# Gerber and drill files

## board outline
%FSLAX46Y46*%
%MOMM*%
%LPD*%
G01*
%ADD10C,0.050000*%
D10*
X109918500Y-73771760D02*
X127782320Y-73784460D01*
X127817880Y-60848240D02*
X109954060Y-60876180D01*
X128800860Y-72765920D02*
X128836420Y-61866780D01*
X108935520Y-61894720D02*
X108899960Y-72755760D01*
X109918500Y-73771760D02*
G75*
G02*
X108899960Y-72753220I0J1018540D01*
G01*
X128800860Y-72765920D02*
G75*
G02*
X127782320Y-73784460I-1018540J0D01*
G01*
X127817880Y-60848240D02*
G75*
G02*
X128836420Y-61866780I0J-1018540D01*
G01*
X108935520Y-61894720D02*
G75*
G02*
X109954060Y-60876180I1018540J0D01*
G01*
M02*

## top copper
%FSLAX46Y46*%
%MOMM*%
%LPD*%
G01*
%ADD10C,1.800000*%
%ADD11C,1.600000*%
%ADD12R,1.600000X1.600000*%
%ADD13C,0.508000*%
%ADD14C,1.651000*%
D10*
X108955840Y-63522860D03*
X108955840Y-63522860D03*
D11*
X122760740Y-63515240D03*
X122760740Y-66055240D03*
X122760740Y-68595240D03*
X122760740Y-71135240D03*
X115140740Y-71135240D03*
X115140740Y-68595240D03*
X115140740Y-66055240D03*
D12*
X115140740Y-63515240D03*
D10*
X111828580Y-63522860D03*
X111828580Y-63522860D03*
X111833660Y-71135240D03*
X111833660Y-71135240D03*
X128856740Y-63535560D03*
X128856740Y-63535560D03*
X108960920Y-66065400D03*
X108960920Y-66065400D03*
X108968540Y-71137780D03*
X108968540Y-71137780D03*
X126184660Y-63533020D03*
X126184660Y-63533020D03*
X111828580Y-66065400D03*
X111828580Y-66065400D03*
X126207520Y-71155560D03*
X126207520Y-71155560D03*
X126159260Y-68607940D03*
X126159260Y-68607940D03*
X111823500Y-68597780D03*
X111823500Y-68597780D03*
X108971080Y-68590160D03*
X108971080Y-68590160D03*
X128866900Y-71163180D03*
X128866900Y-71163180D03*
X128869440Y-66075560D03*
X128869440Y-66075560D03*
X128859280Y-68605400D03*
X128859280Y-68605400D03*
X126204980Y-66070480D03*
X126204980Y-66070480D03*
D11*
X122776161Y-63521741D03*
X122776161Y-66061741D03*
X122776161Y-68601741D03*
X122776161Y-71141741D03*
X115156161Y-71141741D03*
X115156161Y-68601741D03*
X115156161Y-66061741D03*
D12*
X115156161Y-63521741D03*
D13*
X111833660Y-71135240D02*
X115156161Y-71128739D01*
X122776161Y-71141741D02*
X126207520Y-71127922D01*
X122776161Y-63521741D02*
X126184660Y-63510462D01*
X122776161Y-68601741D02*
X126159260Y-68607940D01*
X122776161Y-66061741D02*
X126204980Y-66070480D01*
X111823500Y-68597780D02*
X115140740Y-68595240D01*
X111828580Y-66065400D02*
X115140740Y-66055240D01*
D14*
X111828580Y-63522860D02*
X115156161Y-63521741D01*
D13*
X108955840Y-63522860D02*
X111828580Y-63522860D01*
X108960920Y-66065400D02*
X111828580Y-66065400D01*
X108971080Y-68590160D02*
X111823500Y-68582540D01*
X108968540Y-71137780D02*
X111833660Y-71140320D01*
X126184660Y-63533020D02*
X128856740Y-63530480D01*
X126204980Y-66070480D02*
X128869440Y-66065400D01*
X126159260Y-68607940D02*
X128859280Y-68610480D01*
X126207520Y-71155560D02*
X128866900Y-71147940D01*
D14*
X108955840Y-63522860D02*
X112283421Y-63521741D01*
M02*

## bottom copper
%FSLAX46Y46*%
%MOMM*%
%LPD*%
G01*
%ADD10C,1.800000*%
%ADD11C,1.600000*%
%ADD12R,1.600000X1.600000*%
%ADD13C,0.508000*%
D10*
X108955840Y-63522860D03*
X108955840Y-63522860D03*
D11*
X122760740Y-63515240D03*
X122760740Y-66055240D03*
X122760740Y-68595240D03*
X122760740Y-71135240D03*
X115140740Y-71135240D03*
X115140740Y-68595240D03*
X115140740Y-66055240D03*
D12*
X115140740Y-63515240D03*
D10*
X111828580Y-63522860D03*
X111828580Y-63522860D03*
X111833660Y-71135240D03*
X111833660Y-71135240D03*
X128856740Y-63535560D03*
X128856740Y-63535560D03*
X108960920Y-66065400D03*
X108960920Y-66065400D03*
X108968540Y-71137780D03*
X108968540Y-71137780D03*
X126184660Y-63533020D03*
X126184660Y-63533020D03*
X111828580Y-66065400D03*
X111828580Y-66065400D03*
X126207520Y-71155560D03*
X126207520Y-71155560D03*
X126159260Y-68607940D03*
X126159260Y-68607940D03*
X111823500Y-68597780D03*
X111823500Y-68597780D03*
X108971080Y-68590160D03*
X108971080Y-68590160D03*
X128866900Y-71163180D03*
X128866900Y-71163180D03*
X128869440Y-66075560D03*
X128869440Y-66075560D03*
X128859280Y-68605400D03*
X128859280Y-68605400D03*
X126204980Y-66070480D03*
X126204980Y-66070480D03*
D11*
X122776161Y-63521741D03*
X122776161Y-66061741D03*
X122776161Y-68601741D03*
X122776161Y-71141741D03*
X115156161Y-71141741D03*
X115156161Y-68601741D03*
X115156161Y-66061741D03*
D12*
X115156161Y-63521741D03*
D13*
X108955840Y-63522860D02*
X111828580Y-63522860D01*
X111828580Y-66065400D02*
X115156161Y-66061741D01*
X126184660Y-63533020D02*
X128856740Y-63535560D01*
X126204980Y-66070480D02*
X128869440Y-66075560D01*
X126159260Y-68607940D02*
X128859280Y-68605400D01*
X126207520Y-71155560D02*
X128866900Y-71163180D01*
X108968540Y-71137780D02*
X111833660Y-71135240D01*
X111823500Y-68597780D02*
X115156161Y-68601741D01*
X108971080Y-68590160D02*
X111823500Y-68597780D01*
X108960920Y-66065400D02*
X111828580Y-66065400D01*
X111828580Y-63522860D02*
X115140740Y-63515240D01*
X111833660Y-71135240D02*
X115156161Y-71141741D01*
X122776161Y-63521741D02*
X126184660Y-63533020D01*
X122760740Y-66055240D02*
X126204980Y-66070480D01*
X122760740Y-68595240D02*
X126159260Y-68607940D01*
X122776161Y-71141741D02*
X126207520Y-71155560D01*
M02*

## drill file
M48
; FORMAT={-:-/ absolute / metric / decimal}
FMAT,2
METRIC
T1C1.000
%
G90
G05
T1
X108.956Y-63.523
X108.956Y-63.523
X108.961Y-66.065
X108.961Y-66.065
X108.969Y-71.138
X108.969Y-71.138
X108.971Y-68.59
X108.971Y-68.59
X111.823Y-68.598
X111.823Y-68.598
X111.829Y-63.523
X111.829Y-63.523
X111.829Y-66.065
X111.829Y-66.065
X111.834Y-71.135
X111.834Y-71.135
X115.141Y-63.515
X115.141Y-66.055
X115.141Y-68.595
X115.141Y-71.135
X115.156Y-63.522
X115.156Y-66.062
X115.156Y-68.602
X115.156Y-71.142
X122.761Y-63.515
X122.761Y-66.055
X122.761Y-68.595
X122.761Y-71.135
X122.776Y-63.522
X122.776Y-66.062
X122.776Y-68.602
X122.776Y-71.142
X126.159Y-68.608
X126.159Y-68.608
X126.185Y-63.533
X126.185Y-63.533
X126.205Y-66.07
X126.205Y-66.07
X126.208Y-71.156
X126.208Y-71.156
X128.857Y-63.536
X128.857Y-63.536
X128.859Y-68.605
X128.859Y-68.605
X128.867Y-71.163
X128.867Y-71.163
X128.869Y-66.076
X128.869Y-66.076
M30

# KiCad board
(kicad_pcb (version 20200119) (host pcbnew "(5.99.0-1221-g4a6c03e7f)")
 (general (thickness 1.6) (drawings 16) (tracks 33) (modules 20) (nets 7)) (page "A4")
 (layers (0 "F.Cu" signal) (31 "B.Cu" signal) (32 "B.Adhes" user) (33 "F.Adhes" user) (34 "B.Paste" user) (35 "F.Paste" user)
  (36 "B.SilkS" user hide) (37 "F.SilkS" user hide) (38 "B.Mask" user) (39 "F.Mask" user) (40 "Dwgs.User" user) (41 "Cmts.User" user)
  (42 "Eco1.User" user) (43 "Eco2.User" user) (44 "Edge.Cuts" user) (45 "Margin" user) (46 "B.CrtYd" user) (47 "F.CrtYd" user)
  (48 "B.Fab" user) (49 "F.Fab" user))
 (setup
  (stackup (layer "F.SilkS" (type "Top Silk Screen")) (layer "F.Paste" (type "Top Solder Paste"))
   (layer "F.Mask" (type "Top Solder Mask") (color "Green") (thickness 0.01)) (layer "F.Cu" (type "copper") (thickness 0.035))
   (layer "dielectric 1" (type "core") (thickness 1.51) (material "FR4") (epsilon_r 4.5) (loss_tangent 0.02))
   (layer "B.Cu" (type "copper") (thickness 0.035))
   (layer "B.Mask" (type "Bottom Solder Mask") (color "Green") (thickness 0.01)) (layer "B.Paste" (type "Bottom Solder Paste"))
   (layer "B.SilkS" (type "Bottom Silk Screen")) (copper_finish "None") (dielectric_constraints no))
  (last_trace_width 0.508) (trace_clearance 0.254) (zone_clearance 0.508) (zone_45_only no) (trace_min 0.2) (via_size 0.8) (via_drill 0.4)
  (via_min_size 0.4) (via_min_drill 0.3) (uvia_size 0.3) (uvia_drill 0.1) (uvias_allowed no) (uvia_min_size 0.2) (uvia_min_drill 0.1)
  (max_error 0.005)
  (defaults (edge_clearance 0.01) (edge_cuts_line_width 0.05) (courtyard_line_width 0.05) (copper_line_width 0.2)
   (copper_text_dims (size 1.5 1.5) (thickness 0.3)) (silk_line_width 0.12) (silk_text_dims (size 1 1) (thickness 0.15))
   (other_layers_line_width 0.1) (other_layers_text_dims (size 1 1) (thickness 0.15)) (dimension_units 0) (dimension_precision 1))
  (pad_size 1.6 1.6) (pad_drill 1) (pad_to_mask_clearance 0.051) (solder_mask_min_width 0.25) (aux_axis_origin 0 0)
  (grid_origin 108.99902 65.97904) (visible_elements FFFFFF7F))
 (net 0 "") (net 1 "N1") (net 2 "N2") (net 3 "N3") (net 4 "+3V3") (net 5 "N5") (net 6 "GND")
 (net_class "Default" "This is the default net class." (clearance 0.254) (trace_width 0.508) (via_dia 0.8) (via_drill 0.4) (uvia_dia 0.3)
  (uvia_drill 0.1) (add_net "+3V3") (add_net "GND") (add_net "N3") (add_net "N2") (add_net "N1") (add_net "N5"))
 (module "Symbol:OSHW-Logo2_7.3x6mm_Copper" (layer "B.Cu") (at 118.97902 67.88904 180)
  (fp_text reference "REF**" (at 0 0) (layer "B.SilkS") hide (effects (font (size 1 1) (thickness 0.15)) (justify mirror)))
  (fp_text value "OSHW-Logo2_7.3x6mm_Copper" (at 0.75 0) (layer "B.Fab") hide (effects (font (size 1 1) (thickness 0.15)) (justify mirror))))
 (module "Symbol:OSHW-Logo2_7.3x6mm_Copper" (layer "F.Cu") (at 118.98122 67.88404)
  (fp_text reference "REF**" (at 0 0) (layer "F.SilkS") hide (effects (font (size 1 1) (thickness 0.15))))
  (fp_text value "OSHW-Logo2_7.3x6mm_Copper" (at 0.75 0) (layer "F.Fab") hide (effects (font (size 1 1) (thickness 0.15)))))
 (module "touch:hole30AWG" (layer "F.Cu") (at 108.95584 63.52286)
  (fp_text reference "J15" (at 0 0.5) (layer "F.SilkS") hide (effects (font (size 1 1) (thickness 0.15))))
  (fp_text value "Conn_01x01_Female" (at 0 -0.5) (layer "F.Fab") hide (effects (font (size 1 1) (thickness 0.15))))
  (pad "1" thru_hole circle (at 0 0) (size 1.8 1.8) (drill 1) (layers "F.Cu" "F.Mask") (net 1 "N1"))
  (pad "1" thru_hole circle (at 0 0) (size 1.8 1.8) (drill 1) (layers "B.Cu" "B.Mask") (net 1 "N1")))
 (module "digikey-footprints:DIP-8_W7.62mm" (layer "F.Cu") (at 115.14074 63.51524)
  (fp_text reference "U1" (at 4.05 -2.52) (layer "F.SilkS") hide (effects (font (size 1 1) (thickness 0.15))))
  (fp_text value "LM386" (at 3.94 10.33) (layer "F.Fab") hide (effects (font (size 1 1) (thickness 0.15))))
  (pad "8" thru_hole circle (at 7.62 0) (size 1.6 1.6) (drill 1) (layers *.Cu *.Mask) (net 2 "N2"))
  (pad "7" thru_hole circle (at 7.62 2.54) (size 1.6 1.6) (drill 1) (layers *.Cu *.Mask) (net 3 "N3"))
  (pad "6" thru_hole circle (at 7.62 5.08) (size 1.6 1.6) (drill 1) (layers *.Cu *.Mask) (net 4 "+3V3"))
  (pad "5" thru_hole circle (at 7.62 7.62) (size 1.6 1.6) (drill 1) (layers *.Cu *.Mask) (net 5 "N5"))
  (pad "4" thru_hole circle (at 0 7.62) (size 1.6 1.6) (drill 1) (layers *.Cu *.Mask) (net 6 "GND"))
  (pad "3" thru_hole circle (at 0 5.08) (size 1.6 1.6) (drill 1) (layers *.Cu *.Mask) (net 4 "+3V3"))
  (pad "2" thru_hole circle (at 0 2.54) (size 1.6 1.6) (drill 1) (layers *.Cu *.Mask) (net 6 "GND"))
  (pad "1" thru_hole rect (at 0 0) (size 1.6 1.6) (drill 1) (layers *.Cu *.Mask) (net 1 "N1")))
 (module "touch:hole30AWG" (layer "F.Cu") (at 111.82858 63.52286)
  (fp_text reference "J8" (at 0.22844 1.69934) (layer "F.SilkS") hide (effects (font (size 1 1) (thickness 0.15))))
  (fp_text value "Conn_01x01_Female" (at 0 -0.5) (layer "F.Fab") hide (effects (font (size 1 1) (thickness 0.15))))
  (pad "1" thru_hole circle (at 0 0) (size 1.8 1.8) (drill 1) (layers "F.Cu" "F.Mask") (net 1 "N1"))
  (pad "1" thru_hole circle (at 0 0) (size 1.8 1.8) (drill 1) (layers "B.Cu" "B.Mask") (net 1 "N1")))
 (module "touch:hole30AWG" (layer "F.Cu") (at 111.83366 71.13524)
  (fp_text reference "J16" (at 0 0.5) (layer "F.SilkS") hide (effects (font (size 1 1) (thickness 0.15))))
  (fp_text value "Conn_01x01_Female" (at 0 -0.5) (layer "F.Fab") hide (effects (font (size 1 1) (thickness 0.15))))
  (pad "1" thru_hole circle (at 0 0) (size 1.8 1.8) (drill 1) (layers "F.Cu" "F.Mask") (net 6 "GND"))
  (pad "1" thru_hole circle (at 0 0) (size 1.8 1.8) (drill 1) (layers "B.Cu" "B.Mask") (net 6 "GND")))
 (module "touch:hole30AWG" (layer "F.Cu") (at 128.85674 63.53556)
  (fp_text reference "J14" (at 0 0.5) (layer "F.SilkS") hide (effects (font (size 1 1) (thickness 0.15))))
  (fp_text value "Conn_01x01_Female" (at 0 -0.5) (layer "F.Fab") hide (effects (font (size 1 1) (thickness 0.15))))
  (pad "1" thru_hole circle (at 0 0) (size 1.8 1.8) (drill 1) (layers "F.Cu" "F.Mask") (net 2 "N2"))
  (pad "1" thru_hole circle (at 0 0) (size 1.8 1.8) (drill 1) (layers "B.Cu" "B.Mask") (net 2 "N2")))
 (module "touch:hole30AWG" (layer "F.Cu") (at 108.96092 66.0654)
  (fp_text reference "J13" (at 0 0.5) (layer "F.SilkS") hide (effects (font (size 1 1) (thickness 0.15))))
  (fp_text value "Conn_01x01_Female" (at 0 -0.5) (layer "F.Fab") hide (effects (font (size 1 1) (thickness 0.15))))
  (pad "1" thru_hole circle (at 0 0) (size 1.8 1.8) (drill 1) (layers "F.Cu" "F.Mask") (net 6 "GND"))
  (pad "1" thru_hole circle (at 0 0) (size 1.8 1.8) (drill 1) (layers "B.Cu" "B.Mask") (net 6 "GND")))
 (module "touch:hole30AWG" (layer "F.Cu") (at 108.96854 71.13778)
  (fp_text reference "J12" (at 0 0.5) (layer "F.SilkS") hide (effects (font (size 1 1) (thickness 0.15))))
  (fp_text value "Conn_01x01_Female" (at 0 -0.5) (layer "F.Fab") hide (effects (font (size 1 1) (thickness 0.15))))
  (pad "1" thru_hole circle (at 0 0) (size 1.8 1.8) (drill 1) (layers "F.Cu" "F.Mask") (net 6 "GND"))
  (pad "1" thru_hole circle (at 0 0) (size 1.8 1.8) (drill 1) (layers "B.Cu" "B.Mask") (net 6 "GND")))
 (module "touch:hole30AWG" (layer "F.Cu") (at 126.18466 63.53302)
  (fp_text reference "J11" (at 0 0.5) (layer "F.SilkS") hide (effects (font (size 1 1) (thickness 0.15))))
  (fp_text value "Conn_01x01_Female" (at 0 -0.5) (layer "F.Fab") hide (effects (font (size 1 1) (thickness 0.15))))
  (pad "1" thru_hole circle (at 0 0) (size 1.8 1.8) (drill 1) (layers "F.Cu" "F.Mask") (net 2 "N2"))
  (pad "1" thru_hole circle (at 0 0) (size 1.8 1.8) (drill 1) (layers "B.Cu" "B.Mask") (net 2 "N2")))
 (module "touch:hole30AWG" (layer "F.Cu") (at 111.82858 66.0654)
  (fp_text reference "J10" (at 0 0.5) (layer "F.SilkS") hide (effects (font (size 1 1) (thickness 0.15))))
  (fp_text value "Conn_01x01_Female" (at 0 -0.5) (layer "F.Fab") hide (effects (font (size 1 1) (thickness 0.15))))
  (pad "1" thru_hole circle (at 0 0) (size 1.8 1.8) (drill 1) (layers "F.Cu" "F.Mask") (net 6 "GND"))
  (pad "1" thru_hole circle (at 0 0) (size 1.8 1.8) (drill 1) (layers "B.Cu" "B.Mask") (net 6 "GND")))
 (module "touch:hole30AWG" (layer "F.Cu") (at 126.20752 71.15556)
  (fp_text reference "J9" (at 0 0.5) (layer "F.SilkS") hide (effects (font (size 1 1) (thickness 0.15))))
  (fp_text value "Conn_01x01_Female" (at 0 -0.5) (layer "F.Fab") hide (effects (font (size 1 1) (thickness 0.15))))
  (pad "1" thru_hole circle (at 0 0) (size 1.8 1.8) (drill 1) (layers "F.Cu" "F.Mask") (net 5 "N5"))
  (pad "1" thru_hole circle (at 0 0) (size 1.8 1.8) (drill 1) (layers "B.Cu" "B.Mask") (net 5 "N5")))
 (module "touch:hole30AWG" (layer "F.Cu") (at 126.15926 68.60794)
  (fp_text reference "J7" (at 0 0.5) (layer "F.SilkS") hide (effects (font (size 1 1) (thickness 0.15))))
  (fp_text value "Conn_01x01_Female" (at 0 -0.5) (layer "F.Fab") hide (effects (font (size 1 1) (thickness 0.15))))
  (pad "1" thru_hole circle (at 0 0) (size 1.8 1.8) (drill 1) (layers "F.Cu" "F.Mask") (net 4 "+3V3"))
  (pad "1" thru_hole circle (at 0 0) (size 1.8 1.8) (drill 1) (layers "B.Cu" "B.Mask") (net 4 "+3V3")))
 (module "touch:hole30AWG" (layer "F.Cu") (at 111.8235 68.59778)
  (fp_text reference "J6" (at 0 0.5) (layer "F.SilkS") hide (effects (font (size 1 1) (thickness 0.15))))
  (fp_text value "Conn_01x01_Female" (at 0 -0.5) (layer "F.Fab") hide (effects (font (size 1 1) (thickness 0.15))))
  (pad "1" thru_hole circle (at 0 0) (size 1.8 1.8) (drill 1) (layers "F.Cu" "F.Mask") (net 4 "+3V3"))
  (pad "1" thru_hole circle (at 0 0) (size 1.8 1.8) (drill 1) (layers "B.Cu" "B.Mask") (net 4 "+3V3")))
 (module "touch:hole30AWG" (layer "F.Cu") (at 108.97108 68.59016)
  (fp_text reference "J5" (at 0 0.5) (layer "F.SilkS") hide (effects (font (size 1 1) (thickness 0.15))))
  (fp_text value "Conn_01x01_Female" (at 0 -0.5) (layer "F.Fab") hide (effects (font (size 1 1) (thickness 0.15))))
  (pad "1" thru_hole circle (at 0 0) (size 1.8 1.8) (drill 1) (layers "F.Cu" "F.Mask") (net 4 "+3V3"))
  (pad "1" thru_hole circle (at 0 0) (size 1.8 1.8) (drill 1) (layers "B.Cu" "B.Mask") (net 4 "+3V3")))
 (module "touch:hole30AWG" (layer "F.Cu") (at 128.8669 71.16318)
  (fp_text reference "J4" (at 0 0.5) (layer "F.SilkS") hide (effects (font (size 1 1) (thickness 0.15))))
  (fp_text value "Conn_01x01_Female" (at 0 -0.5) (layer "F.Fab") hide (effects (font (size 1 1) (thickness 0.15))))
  (pad "1" thru_hole circle (at 0 0) (size 1.8 1.8) (drill 1) (layers "F.Cu" "F.Mask") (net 5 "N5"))
  (pad "1" thru_hole circle (at 0 0) (size 1.8 1.8) (drill 1) (layers "B.Cu" "B.Mask") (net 5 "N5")))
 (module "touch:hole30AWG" (layer "F.Cu") (at 128.86944 66.07556)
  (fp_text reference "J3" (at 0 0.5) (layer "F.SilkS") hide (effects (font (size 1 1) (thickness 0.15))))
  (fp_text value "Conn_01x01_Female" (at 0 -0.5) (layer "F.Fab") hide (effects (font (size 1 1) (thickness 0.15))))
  (pad "1" thru_hole circle (at 0 0) (size 1.8 1.8) (drill 1) (layers "F.Cu" "F.Mask") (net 3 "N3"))
  (pad "1" thru_hole circle (at 0 0) (size 1.8 1.8) (drill 1) (layers "B.Cu" "B.Mask") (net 3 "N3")))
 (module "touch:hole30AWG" (layer "F.Cu") (at 128.85928 68.6054)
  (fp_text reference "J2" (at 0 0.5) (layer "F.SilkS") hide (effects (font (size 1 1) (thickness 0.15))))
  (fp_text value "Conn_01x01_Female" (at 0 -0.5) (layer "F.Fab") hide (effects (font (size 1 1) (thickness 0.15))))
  (pad "1" thru_hole circle (at 0 0) (size 1.8 1.8) (drill 1) (layers "F.Cu" "F.Mask") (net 4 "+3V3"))
  (pad "1" thru_hole circle (at 0 0) (size 1.8 1.8) (drill 1) (layers "B.Cu" "B.Mask") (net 4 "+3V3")))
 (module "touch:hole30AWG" (layer "F.Cu") (at 126.20498 66.07048)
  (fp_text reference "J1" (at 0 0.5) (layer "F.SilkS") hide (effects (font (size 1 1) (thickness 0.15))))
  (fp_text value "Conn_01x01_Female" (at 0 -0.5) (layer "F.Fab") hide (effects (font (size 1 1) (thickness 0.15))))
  (pad "1" thru_hole circle (at 0 0) (size 1.8 1.8) (drill 1) (layers "F.Cu" "F.Mask") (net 3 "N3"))
  (pad "1" thru_hole circle (at 0 0) (size 1.8 1.8) (drill 1) (layers "B.Cu" "B.Mask") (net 3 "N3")))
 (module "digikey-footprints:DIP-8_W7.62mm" (layer "F.Cu") (at 115.156161 63.521741)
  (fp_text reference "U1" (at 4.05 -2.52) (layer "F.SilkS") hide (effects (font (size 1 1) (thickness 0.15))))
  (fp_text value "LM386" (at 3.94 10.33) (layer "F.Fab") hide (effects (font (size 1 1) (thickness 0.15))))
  (pad "8" thru_hole circle (at 7.62 0) (size 1.6 1.6) (drill 1) (layers *.Cu *.Mask) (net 2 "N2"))
  (pad "7" thru_hole circle (at 7.62 2.54) (size 1.6 1.6) (drill 1) (layers *.Cu *.Mask) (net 3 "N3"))
  (pad "6" thru_hole circle (at 7.62 5.08) (size 1.6 1.6) (drill 1) (layers *.Cu *.Mask) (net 4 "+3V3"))
  (pad "5" thru_hole circle (at 7.62 7.62) (size 1.6 1.6) (drill 1) (layers *.Cu *.Mask) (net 5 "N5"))
  (pad "4" thru_hole circle (at 0 7.62) (size 1.6 1.6) (drill 1) (layers *.Cu *.Mask) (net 6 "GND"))
  (pad "3" thru_hole circle (at 0 5.08) (size 1.6 1.6) (drill 1) (layers *.Cu *.Mask) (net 4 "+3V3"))
  (pad "2" thru_hole circle (at 0 2.54) (size 1.6 1.6) (drill 1) (layers *.Cu *.Mask) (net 6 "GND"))
  (pad "1" thru_hole rect (at 0 0) (size 1.6 1.6) (drill 1) (layers *.Cu *.Mask) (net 1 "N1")))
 (gr_line (start 109.9185 73.77176) (end 127.78232 73.78446) (layer "Edge.Cuts") (width 0.05))
 (gr_line (start 127.81788 60.84824) (end 109.95406 60.87618) (layer "Edge.Cuts") (width 0.05))
 (gr_line (start 128.80086 72.76592) (end 128.83642 61.86678) (layer "Edge.Cuts") (width 0.05))
 (gr_line (start 108.93552 61.89472) (end 108.89996 72.75576) (layer "Edge.Cuts") (width 0.05))
 (gr_arc (start 109.9185 72.75322) (end 108.89996 72.75322) (angle -90) (layer "Edge.Cuts") (width 0.05))
 (gr_arc (start 127.78232 72.76592) (end 127.78232 73.78446) (angle -90) (layer "Edge.Cuts") (width 0.05))
 (gr_arc (start 127.81788 61.86678) (end 128.83642 61.86678) (angle -90) (layer "Edge.Cuts") (width 0.05))
 (gr_arc (start 109.95406 61.89472) (end 109.95406 60.87618) (angle -90) (layer "Edge.Cuts") (width 0.05))
 (segment (start 111.83366 71.13524) (end 115.156161 71.128739) (width 0.508) (layer "F.Cu") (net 6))
 (segment (start 122.776161 71.141741) (end 126.20752 71.127922) (width 0.508) (layer "F.Cu") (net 5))
 (segment (start 122.776161 63.521741) (end 126.18466 63.510462) (width 0.508) (layer "F.Cu") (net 2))
 (segment (start 122.776161 68.601741) (end 126.15926 68.60794) (width 0.508) (layer "F.Cu") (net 4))
 (segment (start 122.776161 66.061741) (end 126.20498 66.07048) (width 0.508) (layer "F.Cu") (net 3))
 (segment (start 111.8235 68.59778) (end 115.14074 68.59524) (width 0.508) (layer "F.Cu") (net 4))
 (segment (start 111.82858 66.0654) (end 115.14074 66.05524) (width 0.508) (layer "F.Cu") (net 6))
 (segment (start 111.82858 63.52286) (end 115.156161 63.521741) (width 1.651) (layer "F.Cu") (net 1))
 (segment (start 108.95584 63.52286) (end 111.82858 63.52286) (width 0.508) (layer "B.Cu") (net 1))
 (segment (start 111.82858 66.0654) (end 115.156161 66.061741) (width 0.508) (layer "B.Cu") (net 6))
 (segment (start 126.18466 63.53302) (end 128.85674 63.53556) (width 0.508) (layer "B.Cu") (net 2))
 (segment (start 126.20498 66.07048) (end 128.86944 66.07556) (width 0.508) (layer "B.Cu") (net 3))
 (segment (start 126.15926 68.60794) (end 128.85928 68.6054) (width 0.508) (layer "B.Cu") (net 4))
 (segment (start 126.20752 71.15556) (end 128.8669 71.16318) (width 0.508) (layer "B.Cu") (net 5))
 (segment (start 108.96854 71.13778) (end 111.83366 71.13524) (width 0.508) (layer "B.Cu") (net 6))
 (segment (start 111.8235 68.59778) (end 115.156161 68.601741) (width 0.508) (layer "B.Cu") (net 4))
 (segment (start 108.97108 68.59016) (end 111.8235 68.59778) (width 0.508) (layer "B.Cu") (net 4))
 (segment (start 108.96092 66.0654) (end 111.82858 66.0654) (width 0.508) (layer "B.Cu") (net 6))
 (segment (start 111.82858 63.52286) (end 115.14074 63.51524) (width 0.508) (layer "B.Cu") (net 1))
 (segment (start 111.83366 71.13524) (end 115.156161 71.141741) (width 0.508) (layer "B.Cu") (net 6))
 (segment (start 122.776161 63.521741) (end 126.18466 63.53302) (width 0.508) (layer "B.Cu") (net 2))
 (segment (start 122.76074 66.05524) (end 126.20498 66.07048) (width 0.508) (layer "B.Cu") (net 3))
 (segment (start 122.76074 68.59524) (end 126.15926 68.60794) (width 0.508) (layer "B.Cu") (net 4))
 (segment (start 122.776161 71.141741) (end 126.20752 71.15556) (width 0.508) (layer "B.Cu") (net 5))
 (segment (start 108.95584 63.52286) (end 111.82858 63.52286) (width 0.508) (layer "F.Cu") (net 1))
 (segment (start 108.96092 66.0654) (end 111.82858 66.0654) (width 0.508) (layer "F.Cu") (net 6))
 (segment (start 108.97108 68.59016) (end 111.8235 68.58254) (width 0.508) (layer "F.Cu") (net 4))
 (segment (start 108.96854 71.13778) (end 111.83366 71.14032) (width 0.508) (layer "F.Cu") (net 6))
 (segment (start 126.18466 63.53302) (end 128.85674 63.53048) (width 0.508) (layer "F.Cu") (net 2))
 (segment (start 126.20498 66.07048) (end 128.86944 66.0654) (width 0.508) (layer "F.Cu") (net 3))
 (segment (start 126.15926 68.60794) (end 128.85928 68.61048) (width 0.508) (layer "F.Cu") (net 4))
 (segment (start 126.20752 71.15556) (end 128.8669 71.14794) (width 0.508) (layer "F.Cu") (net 5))
 (segment (start 108.95584 63.52286) (end 112.283421 63.521741) (width 1.651) (layer "F.Cu") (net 1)))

